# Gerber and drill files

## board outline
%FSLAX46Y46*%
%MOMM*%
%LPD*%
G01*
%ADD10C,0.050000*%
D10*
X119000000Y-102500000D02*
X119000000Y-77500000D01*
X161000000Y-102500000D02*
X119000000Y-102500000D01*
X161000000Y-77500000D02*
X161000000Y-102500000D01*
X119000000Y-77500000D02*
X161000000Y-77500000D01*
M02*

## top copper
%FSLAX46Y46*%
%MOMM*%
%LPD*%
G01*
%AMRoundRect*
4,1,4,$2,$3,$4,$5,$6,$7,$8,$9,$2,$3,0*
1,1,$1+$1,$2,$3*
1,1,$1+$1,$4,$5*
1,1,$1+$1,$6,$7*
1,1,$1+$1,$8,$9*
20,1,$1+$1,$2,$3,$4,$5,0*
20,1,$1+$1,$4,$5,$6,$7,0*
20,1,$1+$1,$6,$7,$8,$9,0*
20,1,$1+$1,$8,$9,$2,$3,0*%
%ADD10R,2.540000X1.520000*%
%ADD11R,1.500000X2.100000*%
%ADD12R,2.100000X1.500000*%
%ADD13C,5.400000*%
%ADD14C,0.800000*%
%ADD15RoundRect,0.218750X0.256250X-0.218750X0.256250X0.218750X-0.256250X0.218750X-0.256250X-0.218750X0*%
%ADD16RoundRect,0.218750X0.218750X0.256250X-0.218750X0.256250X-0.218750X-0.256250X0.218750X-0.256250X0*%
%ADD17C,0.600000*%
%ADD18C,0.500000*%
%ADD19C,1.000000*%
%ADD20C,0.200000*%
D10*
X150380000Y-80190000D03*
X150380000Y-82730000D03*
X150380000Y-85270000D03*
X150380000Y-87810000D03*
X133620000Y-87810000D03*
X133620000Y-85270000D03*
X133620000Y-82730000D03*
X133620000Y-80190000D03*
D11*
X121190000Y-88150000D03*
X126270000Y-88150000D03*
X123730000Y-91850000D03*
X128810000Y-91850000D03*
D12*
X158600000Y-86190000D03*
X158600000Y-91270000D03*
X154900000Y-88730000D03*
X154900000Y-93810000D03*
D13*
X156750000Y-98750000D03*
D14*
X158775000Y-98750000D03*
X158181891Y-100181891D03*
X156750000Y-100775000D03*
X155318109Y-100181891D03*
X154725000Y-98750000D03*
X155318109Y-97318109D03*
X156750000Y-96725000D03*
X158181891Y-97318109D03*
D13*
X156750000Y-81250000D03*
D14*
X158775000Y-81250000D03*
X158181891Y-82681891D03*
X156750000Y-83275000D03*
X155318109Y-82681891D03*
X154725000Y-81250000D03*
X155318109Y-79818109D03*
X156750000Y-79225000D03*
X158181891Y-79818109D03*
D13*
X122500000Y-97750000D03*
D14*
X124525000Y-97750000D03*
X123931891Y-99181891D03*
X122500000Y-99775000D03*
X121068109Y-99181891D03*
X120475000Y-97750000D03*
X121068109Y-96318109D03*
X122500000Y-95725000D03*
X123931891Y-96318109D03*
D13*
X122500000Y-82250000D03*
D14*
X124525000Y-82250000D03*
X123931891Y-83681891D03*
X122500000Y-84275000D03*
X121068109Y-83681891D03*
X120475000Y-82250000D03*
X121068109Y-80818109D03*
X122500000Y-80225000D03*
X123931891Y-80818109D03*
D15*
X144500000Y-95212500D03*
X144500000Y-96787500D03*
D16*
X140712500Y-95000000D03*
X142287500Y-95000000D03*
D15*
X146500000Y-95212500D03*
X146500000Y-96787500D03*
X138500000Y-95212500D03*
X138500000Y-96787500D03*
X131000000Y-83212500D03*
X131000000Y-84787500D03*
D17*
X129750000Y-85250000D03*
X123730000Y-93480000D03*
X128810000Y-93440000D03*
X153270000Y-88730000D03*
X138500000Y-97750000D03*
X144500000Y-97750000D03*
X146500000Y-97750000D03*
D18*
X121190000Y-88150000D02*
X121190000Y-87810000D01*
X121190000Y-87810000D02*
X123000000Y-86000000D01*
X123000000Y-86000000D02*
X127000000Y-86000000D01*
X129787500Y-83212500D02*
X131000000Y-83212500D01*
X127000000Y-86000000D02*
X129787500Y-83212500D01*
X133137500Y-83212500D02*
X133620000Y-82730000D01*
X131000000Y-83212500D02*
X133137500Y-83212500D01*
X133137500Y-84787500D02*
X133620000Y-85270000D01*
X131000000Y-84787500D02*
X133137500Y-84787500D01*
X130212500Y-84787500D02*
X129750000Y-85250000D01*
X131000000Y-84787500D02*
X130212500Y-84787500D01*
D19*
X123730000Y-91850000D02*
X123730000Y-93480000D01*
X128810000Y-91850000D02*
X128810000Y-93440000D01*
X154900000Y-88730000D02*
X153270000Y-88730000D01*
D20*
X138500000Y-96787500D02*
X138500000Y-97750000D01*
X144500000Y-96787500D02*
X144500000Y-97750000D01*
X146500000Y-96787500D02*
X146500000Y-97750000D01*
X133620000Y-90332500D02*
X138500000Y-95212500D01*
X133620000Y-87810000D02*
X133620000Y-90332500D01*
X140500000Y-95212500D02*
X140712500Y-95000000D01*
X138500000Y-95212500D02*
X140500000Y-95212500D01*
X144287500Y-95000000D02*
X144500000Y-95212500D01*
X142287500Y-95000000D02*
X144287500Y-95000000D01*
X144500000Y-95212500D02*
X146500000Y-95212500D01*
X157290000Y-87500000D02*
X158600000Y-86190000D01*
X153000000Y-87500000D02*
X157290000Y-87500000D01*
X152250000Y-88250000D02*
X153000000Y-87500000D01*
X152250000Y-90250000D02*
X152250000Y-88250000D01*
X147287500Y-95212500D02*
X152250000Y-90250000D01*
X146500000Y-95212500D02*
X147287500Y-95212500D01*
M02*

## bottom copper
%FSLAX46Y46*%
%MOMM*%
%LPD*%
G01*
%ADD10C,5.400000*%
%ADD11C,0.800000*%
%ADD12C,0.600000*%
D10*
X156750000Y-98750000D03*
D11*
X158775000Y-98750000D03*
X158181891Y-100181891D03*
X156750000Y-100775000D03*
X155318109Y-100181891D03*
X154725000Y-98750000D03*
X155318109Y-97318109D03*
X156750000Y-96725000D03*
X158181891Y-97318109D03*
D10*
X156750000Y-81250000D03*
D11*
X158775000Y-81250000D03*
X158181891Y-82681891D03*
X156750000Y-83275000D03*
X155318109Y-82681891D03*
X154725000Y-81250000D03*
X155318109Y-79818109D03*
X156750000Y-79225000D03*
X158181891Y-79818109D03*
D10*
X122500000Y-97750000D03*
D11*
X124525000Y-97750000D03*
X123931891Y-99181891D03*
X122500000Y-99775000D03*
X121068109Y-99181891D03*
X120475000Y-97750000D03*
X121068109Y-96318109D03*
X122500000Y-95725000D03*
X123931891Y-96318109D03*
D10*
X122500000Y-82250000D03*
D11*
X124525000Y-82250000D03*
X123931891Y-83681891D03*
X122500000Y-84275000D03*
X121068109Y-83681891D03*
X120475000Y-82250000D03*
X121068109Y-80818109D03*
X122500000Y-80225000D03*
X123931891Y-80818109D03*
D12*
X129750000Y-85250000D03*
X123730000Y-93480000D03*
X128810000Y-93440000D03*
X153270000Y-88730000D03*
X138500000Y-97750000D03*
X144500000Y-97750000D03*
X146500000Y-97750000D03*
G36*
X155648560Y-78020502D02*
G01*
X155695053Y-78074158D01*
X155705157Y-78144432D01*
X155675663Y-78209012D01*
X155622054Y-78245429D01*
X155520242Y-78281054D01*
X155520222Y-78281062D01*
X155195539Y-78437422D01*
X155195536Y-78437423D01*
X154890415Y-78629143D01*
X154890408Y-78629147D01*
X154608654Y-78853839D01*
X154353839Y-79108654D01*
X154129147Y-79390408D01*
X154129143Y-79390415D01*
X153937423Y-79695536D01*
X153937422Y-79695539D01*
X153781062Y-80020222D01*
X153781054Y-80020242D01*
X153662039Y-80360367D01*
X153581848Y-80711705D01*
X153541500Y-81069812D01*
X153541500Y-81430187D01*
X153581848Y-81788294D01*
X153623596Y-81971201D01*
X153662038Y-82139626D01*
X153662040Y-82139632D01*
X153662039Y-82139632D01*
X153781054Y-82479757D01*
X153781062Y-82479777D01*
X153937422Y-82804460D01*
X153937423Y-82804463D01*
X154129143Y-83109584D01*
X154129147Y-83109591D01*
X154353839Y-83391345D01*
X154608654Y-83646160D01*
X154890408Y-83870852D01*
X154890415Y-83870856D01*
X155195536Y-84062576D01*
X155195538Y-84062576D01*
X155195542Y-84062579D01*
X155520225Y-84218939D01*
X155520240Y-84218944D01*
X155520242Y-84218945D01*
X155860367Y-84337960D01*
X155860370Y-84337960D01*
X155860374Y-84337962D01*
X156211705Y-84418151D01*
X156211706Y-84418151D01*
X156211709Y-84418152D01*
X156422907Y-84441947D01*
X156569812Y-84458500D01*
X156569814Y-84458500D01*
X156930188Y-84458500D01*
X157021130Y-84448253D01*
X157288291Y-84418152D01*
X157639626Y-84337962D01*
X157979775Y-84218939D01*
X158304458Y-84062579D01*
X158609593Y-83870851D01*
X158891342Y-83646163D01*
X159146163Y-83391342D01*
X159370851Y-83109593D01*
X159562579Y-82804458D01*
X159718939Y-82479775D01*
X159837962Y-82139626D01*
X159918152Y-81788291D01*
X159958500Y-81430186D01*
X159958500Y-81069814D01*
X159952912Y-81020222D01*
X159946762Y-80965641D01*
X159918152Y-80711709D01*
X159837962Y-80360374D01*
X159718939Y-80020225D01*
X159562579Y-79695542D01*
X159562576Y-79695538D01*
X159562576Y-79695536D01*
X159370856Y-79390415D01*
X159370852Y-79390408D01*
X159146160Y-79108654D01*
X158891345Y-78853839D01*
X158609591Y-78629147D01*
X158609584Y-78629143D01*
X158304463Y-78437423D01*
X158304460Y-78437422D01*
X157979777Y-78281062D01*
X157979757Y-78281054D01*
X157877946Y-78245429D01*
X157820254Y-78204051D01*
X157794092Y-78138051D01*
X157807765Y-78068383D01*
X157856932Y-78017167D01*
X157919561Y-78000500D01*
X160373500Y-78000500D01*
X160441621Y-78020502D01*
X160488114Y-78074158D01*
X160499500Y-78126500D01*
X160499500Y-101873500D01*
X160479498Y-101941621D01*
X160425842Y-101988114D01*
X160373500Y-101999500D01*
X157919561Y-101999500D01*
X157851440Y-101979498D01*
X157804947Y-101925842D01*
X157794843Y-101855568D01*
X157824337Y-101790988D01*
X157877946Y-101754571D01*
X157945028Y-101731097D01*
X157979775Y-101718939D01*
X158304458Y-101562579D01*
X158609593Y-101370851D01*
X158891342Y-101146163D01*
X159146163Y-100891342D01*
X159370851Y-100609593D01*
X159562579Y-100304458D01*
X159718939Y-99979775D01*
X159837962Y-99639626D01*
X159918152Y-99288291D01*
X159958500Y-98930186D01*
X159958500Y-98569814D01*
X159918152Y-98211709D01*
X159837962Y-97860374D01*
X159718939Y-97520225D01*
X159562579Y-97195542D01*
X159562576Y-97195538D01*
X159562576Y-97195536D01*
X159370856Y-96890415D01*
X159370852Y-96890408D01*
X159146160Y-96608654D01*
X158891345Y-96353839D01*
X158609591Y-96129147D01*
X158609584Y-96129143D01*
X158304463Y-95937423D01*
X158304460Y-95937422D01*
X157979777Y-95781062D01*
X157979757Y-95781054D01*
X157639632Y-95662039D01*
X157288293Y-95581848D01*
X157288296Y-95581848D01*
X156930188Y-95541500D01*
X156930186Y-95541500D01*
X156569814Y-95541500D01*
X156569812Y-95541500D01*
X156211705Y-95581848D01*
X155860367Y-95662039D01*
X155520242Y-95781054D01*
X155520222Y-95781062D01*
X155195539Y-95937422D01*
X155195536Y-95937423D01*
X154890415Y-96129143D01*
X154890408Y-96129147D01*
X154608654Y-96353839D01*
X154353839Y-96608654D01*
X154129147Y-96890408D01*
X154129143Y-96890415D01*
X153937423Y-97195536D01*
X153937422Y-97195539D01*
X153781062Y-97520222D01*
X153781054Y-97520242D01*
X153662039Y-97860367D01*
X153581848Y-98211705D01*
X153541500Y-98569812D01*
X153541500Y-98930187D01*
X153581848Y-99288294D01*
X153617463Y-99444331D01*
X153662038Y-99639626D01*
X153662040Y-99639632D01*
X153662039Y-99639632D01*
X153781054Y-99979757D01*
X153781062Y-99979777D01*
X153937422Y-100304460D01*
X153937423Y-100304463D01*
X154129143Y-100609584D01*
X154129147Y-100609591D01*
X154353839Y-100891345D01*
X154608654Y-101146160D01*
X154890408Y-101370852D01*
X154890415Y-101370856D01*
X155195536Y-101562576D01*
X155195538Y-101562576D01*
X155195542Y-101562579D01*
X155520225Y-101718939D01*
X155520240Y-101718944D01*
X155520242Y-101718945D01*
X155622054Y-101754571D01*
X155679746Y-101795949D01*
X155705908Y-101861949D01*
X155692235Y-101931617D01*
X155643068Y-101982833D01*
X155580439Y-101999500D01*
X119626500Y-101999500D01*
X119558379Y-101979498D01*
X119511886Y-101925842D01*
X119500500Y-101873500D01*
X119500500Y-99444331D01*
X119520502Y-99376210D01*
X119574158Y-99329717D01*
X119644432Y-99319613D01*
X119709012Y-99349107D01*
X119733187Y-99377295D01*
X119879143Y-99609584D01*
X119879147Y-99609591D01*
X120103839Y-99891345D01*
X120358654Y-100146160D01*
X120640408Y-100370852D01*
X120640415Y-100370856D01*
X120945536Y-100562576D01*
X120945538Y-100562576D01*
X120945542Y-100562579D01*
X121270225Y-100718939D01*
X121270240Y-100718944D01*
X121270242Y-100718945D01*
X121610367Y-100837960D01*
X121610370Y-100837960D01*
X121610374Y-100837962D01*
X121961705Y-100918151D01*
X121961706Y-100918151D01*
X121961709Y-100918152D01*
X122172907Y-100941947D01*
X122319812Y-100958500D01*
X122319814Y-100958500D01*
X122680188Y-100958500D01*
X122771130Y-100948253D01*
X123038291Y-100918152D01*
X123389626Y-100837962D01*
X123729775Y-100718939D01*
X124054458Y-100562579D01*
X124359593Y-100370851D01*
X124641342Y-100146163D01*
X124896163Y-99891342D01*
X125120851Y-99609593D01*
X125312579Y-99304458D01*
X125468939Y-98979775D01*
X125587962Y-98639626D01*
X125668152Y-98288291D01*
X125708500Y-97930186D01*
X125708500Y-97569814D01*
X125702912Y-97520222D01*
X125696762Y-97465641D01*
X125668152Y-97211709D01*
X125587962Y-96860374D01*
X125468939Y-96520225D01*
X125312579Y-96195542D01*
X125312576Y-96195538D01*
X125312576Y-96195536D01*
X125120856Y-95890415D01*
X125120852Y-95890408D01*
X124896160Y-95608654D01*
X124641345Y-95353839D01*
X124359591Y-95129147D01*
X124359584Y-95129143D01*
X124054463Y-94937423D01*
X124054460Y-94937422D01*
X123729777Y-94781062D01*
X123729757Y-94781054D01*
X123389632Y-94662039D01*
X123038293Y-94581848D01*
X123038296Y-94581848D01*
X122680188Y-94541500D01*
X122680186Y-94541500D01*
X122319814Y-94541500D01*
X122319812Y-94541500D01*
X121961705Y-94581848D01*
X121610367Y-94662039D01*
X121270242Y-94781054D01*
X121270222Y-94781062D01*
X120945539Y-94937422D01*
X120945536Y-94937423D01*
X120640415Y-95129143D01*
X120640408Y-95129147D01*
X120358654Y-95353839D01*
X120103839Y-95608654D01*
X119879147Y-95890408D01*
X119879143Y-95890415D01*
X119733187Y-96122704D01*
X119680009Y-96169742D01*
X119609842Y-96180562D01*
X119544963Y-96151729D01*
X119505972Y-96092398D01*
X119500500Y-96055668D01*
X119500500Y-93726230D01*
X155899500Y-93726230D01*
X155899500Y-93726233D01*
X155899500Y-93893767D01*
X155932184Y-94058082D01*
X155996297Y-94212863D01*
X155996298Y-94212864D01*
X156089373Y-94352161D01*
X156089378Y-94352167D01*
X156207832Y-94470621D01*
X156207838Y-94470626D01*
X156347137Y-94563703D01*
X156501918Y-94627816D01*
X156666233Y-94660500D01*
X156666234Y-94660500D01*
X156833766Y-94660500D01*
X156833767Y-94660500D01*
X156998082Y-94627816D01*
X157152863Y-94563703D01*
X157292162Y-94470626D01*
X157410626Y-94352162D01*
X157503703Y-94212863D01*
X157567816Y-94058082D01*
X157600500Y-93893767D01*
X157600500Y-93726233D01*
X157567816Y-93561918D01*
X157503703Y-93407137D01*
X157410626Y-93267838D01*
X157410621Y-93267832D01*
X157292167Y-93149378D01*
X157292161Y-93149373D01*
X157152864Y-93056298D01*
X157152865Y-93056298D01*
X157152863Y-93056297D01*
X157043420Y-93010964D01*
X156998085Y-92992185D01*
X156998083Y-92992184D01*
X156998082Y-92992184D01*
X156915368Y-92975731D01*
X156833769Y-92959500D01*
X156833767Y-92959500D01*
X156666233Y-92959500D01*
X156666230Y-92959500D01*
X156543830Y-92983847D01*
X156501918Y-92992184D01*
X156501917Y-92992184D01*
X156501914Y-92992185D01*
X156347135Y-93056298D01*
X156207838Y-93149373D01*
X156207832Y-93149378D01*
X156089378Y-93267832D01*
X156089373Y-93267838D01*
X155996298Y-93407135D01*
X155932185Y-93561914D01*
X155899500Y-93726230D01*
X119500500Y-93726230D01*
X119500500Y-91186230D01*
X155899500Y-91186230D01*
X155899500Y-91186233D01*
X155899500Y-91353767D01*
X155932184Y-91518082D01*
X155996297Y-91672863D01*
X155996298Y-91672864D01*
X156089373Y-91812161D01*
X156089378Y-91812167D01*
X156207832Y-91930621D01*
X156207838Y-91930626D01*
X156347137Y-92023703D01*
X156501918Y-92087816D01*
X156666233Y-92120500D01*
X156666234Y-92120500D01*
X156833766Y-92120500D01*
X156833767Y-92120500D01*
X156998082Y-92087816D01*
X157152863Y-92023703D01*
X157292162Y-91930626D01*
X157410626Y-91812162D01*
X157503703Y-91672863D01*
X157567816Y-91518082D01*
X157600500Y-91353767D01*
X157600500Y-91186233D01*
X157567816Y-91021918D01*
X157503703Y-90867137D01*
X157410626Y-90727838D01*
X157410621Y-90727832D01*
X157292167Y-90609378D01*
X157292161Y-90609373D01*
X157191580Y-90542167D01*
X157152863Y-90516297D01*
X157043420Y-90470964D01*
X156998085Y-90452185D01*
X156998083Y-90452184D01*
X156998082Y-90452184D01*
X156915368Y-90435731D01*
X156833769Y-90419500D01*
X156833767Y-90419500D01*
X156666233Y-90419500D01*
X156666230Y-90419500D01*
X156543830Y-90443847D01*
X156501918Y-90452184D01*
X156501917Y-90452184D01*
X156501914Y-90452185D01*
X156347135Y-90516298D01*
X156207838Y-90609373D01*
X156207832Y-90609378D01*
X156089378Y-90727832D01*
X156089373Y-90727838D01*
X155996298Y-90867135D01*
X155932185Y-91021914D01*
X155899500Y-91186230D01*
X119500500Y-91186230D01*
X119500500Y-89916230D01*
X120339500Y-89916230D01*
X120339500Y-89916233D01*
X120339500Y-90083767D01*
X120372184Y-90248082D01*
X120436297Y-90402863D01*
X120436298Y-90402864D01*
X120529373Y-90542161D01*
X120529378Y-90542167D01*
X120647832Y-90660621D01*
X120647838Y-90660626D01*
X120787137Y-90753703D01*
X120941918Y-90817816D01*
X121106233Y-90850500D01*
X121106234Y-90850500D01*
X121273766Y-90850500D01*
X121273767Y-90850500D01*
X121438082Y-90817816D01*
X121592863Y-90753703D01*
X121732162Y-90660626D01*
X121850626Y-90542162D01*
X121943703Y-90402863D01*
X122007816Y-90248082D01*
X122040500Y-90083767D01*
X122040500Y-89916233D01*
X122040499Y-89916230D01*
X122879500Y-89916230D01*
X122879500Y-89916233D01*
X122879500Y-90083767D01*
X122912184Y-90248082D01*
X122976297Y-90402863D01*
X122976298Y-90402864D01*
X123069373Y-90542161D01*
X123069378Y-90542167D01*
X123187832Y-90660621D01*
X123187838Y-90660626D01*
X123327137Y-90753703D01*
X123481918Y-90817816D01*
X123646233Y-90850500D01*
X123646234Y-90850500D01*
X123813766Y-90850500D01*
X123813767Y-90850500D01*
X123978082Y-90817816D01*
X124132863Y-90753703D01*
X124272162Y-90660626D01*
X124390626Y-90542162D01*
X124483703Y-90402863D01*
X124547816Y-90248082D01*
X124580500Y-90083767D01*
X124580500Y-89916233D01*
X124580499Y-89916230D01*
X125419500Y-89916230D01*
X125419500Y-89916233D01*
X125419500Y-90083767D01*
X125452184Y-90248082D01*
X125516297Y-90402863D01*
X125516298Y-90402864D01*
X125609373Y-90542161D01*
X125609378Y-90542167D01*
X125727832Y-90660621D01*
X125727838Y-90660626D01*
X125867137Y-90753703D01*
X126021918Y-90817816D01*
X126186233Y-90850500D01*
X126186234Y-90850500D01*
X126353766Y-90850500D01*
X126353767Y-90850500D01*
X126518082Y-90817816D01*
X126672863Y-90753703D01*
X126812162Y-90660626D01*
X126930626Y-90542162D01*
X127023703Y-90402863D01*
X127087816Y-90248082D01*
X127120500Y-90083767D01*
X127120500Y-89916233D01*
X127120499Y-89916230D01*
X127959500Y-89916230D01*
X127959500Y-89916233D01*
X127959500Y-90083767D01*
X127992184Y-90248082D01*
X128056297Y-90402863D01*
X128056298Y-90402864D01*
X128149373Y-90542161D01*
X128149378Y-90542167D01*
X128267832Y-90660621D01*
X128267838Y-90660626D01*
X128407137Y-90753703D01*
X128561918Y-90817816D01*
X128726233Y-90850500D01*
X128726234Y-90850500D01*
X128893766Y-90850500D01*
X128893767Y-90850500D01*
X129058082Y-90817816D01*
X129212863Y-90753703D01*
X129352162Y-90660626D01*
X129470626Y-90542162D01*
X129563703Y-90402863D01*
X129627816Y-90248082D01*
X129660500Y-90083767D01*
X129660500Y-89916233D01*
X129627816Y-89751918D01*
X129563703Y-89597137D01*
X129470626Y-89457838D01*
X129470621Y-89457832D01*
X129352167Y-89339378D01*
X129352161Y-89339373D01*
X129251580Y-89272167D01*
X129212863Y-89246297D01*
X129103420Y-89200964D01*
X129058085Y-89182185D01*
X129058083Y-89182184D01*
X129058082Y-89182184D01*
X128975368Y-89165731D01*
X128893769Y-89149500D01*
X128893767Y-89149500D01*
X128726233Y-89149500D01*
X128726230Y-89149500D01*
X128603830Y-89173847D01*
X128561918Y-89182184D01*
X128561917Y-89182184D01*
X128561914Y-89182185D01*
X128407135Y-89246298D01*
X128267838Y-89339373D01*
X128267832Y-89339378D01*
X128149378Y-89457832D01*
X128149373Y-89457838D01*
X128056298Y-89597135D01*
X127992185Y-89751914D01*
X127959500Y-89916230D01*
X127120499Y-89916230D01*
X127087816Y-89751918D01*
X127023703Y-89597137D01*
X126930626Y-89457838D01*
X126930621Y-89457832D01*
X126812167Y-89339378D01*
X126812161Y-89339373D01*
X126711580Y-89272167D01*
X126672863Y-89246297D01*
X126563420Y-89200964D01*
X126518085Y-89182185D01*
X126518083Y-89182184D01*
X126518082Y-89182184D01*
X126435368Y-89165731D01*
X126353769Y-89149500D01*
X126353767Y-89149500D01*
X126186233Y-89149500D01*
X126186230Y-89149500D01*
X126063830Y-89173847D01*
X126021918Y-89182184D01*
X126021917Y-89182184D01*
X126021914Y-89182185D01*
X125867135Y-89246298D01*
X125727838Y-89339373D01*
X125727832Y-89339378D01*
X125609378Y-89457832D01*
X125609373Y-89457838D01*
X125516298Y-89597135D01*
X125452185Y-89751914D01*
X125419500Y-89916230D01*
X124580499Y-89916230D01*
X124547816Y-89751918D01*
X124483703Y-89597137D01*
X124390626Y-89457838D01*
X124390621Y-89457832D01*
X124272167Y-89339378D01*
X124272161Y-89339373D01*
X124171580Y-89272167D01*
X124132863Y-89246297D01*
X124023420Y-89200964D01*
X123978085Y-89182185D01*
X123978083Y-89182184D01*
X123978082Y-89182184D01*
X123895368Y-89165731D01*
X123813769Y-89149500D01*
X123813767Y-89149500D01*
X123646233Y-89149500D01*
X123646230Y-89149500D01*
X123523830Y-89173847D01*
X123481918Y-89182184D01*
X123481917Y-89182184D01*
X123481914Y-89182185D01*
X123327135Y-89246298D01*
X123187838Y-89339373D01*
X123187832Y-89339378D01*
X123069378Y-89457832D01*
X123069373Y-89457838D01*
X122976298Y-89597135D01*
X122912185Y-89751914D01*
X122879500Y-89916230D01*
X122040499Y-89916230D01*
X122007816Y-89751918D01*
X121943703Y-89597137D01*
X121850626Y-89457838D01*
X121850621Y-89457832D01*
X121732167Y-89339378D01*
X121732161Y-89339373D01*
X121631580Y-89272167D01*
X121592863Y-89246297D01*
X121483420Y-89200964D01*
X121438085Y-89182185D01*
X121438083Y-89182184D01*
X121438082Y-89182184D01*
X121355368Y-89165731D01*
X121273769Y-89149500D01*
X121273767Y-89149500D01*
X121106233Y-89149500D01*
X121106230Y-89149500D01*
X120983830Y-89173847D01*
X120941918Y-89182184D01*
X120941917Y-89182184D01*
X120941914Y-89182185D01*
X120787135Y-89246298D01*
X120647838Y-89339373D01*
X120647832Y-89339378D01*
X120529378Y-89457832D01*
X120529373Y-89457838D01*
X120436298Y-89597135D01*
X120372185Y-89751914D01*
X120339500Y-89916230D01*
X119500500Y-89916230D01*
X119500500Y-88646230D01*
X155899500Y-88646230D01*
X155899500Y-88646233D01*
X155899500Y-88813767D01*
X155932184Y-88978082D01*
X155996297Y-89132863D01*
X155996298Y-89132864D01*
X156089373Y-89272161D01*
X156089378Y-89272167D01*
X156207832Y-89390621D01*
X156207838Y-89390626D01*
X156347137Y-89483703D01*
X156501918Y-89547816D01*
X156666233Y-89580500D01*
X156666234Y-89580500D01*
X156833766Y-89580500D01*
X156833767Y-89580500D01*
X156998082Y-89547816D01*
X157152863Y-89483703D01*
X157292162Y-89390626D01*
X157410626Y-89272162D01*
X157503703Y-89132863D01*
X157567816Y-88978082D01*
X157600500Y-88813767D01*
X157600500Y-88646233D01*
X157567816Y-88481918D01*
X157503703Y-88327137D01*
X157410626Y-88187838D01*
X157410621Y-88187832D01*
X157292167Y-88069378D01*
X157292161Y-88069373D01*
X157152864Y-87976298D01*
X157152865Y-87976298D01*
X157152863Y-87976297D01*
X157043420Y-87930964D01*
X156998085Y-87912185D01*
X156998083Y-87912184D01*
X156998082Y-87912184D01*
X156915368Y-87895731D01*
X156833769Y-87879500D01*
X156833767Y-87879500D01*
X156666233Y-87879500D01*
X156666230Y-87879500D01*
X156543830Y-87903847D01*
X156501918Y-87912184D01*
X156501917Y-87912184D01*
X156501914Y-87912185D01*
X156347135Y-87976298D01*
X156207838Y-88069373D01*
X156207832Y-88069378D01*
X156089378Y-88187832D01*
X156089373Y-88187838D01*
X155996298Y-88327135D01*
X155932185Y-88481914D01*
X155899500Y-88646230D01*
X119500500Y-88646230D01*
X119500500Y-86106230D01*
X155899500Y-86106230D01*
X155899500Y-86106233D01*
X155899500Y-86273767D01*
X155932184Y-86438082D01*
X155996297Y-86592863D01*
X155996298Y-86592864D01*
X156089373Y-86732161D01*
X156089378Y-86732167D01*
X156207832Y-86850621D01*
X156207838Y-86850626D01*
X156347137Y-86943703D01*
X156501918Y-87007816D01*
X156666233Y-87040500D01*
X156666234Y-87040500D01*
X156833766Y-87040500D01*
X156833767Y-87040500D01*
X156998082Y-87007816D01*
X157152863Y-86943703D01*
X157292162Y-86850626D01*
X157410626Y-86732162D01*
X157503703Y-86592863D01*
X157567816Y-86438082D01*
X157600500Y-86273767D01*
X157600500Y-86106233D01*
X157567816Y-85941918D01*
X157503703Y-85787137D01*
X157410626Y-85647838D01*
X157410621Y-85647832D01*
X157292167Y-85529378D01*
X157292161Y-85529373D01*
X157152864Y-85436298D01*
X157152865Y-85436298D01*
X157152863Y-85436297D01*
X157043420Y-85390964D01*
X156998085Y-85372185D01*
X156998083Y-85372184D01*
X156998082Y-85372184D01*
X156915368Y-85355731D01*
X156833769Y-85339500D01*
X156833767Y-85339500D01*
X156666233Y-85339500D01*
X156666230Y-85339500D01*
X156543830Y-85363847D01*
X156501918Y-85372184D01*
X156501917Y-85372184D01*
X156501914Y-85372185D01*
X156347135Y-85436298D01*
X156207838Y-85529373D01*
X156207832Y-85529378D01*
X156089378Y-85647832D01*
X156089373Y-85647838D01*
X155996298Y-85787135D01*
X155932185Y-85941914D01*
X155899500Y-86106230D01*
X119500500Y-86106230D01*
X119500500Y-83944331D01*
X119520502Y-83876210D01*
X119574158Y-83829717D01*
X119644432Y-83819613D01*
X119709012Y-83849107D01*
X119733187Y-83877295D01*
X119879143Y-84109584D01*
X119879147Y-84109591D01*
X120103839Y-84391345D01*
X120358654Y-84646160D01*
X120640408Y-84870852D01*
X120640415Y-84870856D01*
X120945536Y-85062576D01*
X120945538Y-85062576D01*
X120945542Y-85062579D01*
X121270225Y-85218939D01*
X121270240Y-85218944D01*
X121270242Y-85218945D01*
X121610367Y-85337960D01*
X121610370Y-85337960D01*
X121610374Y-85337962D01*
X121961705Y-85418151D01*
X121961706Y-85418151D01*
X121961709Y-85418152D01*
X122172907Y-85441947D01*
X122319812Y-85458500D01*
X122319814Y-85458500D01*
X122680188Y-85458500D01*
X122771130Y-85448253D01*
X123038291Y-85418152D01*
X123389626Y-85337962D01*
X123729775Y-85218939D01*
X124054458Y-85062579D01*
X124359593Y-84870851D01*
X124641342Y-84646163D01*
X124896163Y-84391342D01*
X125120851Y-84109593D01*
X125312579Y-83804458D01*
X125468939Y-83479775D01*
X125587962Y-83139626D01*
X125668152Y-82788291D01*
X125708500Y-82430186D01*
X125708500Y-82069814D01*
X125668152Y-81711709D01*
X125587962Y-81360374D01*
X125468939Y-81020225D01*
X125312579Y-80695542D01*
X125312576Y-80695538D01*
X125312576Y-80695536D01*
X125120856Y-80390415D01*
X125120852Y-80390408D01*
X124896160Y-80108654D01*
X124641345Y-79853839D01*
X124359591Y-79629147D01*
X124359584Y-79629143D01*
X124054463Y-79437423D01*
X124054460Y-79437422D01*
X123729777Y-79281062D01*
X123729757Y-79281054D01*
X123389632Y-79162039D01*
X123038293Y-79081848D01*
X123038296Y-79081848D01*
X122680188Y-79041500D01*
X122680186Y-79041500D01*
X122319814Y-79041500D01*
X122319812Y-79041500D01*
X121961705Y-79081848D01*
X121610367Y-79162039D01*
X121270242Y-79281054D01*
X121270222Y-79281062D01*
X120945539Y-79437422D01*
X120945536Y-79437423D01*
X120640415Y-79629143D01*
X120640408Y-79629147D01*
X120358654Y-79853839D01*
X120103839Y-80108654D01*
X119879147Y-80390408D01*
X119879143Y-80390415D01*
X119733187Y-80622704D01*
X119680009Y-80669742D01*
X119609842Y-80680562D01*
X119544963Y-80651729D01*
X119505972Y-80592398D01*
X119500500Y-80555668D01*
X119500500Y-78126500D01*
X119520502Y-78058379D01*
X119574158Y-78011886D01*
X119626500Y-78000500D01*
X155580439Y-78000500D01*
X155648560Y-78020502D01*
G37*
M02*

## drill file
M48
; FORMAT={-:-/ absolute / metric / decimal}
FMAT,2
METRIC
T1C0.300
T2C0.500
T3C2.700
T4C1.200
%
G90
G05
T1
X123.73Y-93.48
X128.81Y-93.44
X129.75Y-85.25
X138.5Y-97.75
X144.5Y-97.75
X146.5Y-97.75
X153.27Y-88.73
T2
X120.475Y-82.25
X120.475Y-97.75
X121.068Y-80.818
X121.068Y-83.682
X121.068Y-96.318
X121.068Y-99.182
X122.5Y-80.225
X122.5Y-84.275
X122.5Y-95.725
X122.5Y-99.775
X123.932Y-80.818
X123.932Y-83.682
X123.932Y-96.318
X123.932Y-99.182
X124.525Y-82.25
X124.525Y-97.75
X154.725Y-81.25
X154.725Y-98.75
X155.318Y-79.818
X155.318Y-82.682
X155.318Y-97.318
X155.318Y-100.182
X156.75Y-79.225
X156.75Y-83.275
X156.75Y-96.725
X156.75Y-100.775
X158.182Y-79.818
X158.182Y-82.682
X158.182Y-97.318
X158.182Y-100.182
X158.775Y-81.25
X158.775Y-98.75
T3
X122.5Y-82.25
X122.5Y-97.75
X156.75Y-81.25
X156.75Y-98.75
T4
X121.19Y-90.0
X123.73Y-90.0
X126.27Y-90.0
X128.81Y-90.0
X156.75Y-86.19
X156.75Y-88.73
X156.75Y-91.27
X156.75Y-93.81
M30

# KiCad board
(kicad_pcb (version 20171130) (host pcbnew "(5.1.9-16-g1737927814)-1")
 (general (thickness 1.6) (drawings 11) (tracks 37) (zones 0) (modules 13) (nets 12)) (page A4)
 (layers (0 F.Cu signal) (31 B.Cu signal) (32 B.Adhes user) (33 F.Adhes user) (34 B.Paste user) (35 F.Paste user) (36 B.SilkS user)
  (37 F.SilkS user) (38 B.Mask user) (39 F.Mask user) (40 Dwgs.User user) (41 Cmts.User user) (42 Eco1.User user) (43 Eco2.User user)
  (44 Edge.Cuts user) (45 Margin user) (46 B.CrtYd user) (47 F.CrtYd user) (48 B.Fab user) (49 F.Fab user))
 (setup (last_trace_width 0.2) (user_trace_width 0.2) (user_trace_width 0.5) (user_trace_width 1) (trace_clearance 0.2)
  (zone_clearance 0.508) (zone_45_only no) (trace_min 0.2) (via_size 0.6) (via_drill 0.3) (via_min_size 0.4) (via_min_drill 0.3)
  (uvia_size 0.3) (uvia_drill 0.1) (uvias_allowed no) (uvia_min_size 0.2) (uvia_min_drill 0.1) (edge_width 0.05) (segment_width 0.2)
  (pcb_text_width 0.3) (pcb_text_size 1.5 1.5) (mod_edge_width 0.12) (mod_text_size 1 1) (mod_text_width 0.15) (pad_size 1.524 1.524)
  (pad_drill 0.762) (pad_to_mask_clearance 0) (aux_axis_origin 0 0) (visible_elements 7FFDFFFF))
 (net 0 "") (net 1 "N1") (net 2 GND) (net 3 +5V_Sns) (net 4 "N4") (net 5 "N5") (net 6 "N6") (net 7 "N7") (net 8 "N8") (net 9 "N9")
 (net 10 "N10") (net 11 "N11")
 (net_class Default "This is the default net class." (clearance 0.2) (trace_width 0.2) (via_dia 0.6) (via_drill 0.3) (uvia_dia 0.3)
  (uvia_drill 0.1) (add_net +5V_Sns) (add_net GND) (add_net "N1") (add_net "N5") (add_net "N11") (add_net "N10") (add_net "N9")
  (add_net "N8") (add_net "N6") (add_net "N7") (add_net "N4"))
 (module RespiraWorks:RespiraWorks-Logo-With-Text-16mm (layer B.Cu) (at 139.5 89.75 180)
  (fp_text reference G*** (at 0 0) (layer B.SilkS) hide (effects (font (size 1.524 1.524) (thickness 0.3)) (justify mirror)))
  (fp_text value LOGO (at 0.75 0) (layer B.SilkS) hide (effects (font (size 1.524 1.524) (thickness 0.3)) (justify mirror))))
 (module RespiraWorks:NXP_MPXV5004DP (layer F.Cu) (at 142 84)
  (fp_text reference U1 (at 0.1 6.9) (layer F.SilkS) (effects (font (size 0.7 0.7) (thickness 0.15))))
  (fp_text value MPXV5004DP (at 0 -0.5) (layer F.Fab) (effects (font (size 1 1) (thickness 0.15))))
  (pad 8 smd rect (at 8.38 -3.81) (size 2.54 1.52) (layers F.Cu F.Paste F.Mask))
  (pad 7 smd rect (at 8.38 -1.27) (size 2.54 1.52) (layers F.Cu F.Paste F.Mask))
  (pad 6 smd rect (at 8.38 1.27) (size 2.54 1.52) (layers F.Cu F.Paste F.Mask))
  (pad 5 smd rect (at 8.38 3.81) (size 2.54 1.52) (layers F.Cu F.Paste F.Mask))
  (pad 4 smd rect (at -8.38 3.81) (size 2.54 1.52) (layers F.Cu F.Paste F.Mask) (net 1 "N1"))
  (pad 3 smd rect (at -8.38 1.27) (size 2.54 1.52) (layers F.Cu F.Paste F.Mask) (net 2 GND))
  (pad 2 smd rect (at -8.38 -1.27) (size 2.54 1.52) (layers F.Cu F.Paste F.Mask) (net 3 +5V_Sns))
  (pad 1 smd rect (at -8.38 -3.81) (size 2.54 1.52) (layers F.Cu F.Paste F.Mask)))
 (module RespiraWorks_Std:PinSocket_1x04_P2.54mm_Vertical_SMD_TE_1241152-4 (layer F.Cu) (at 125 90 90)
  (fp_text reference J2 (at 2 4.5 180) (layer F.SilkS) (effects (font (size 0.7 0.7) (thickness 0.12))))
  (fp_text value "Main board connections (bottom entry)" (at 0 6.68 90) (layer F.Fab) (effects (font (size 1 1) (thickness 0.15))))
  (pad "" np_thru_hole circle (at 0 1.27 90) (size 1.2 1.2) (drill 1.2) (layers *.Cu *.Mask))
  (pad "" np_thru_hole circle (at 0 -1.27 90) (size 1.2 1.2) (drill 1.2) (layers *.Cu *.Mask))
  (pad "" np_thru_hole circle (at 0 -3.81 90) (size 1.2 1.2) (drill 1.2) (layers *.Cu *.Mask))
  (pad 1 smd rect (at 1.85 -3.81 90) (size 2.1 1.5) (layers F.Cu F.Paste F.Mask) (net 3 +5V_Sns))
  (pad 3 smd rect (at 1.85 1.27 90) (size 2.1 1.5) (layers F.Cu F.Paste F.Mask) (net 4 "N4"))
  (pad 2 smd rect (at -1.85 -1.27 90) (size 2.1 1.5) (layers F.Cu F.Paste F.Mask) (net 2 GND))
  (pad 4 smd rect (at -1.85 3.81 90) (size 2.1 1.5) (layers F.Cu F.Paste F.Mask) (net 2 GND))
  (pad "" np_thru_hole circle (at 0 3.81 90) (size 1.2 1.2) (drill 1.2) (layers *.Cu *.Mask)))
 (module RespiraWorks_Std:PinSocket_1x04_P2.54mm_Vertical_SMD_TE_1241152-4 (layer F.Cu) (at 156.75 90)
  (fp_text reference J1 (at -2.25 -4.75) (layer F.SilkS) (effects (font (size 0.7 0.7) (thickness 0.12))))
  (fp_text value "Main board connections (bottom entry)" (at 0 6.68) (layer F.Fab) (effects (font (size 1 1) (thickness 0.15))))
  (pad "" np_thru_hole circle (at 0 1.27) (size 1.2 1.2) (drill 1.2) (layers *.Cu *.Mask))
  (pad "" np_thru_hole circle (at 0 -1.27) (size 1.2 1.2) (drill 1.2) (layers *.Cu *.Mask))
  (pad "" np_thru_hole circle (at 0 -3.81) (size 1.2 1.2) (drill 1.2) (layers *.Cu *.Mask))
  (pad 1 smd rect (at 1.85 -3.81) (size 2.1 1.5) (layers F.Cu F.Paste F.Mask) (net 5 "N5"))
  (pad 3 smd rect (at 1.85 1.27) (size 2.1 1.5) (layers F.Cu F.Paste F.Mask) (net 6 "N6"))
  (pad 2 smd rect (at -1.85 -1.27) (size 2.1 1.5) (layers F.Cu F.Paste F.Mask) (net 2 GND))
  (pad 4 smd rect (at -1.85 3.81) (size 2.1 1.5) (layers F.Cu F.Paste F.Mask) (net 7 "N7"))
  (pad "" np_thru_hole circle (at 0 3.81) (size 1.2 1.2) (drill 1.2) (layers *.Cu *.Mask)))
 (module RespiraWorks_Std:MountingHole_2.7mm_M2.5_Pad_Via (layer F.Cu) (at 156.75 98.75)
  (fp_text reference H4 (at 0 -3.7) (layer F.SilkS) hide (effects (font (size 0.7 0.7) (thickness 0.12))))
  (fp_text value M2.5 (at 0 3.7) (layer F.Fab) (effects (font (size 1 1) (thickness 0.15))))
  (pad 1 thru_hole circle (at 0 0) (size 5.4 5.4) (drill 2.7) (layers *.Cu *.Mask) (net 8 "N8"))
  (pad 1 thru_hole circle (at 2.025 0) (size 0.8 0.8) (drill 0.5) (layers *.Cu *.Mask) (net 8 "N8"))
  (pad 1 thru_hole circle (at 1.431891 1.431891) (size 0.8 0.8) (drill 0.5) (layers *.Cu *.Mask) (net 8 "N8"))
  (pad 1 thru_hole circle (at 0 2.025) (size 0.8 0.8) (drill 0.5) (layers *.Cu *.Mask) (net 8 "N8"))
  (pad 1 thru_hole circle (at -1.431891 1.431891) (size 0.8 0.8) (drill 0.5) (layers *.Cu *.Mask) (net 8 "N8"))
  (pad 1 thru_hole circle (at -2.025 0) (size 0.8 0.8) (drill 0.5) (layers *.Cu *.Mask) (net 8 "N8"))
  (pad 1 thru_hole circle (at -1.431891 -1.431891) (size 0.8 0.8) (drill 0.5) (layers *.Cu *.Mask) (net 8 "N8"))
  (pad 1 thru_hole circle (at 0 -2.025) (size 0.8 0.8) (drill 0.5) (layers *.Cu *.Mask) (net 8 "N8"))
  (pad 1 thru_hole circle (at 1.431891 -1.431891) (size 0.8 0.8) (drill 0.5) (layers *.Cu *.Mask) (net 8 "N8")))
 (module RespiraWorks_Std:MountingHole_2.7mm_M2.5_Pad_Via (layer F.Cu) (at 156.75 81.25)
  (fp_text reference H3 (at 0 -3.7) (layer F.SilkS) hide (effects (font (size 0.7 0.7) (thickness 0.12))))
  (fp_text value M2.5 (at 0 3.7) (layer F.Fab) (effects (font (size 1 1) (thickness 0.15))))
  (pad 1 thru_hole circle (at 0 0) (size 5.4 5.4) (drill 2.7) (layers *.Cu *.Mask) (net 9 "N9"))
  (pad 1 thru_hole circle (at 2.025 0) (size 0.8 0.8) (drill 0.5) (layers *.Cu *.Mask) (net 9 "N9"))
  (pad 1 thru_hole circle (at 1.431891 1.431891) (size 0.8 0.8) (drill 0.5) (layers *.Cu *.Mask) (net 9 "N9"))
  (pad 1 thru_hole circle (at 0 2.025) (size 0.8 0.8) (drill 0.5) (layers *.Cu *.Mask) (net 9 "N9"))
  (pad 1 thru_hole circle (at -1.431891 1.431891) (size 0.8 0.8) (drill 0.5) (layers *.Cu *.Mask) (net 9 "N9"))
  (pad 1 thru_hole circle (at -2.025 0) (size 0.8 0.8) (drill 0.5) (layers *.Cu *.Mask) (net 9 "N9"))
  (pad 1 thru_hole circle (at -1.431891 -1.431891) (size 0.8 0.8) (drill 0.5) (layers *.Cu *.Mask) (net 9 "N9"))
  (pad 1 thru_hole circle (at 0 -2.025) (size 0.8 0.8) (drill 0.5) (layers *.Cu *.Mask) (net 9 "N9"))
  (pad 1 thru_hole circle (at 1.431891 -1.431891) (size 0.8 0.8) (drill 0.5) (layers *.Cu *.Mask) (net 9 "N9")))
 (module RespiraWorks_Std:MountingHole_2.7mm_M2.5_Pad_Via (layer F.Cu) (at 122.5 97.75)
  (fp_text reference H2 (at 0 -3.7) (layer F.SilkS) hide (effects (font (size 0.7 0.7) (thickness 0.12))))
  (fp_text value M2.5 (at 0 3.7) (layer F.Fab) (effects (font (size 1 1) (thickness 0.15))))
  (pad 1 thru_hole circle (at 0 0) (size 5.4 5.4) (drill 2.7) (layers *.Cu *.Mask) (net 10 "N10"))
  (pad 1 thru_hole circle (at 2.025 0) (size 0.8 0.8) (drill 0.5) (layers *.Cu *.Mask) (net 10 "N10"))
  (pad 1 thru_hole circle (at 1.431891 1.431891) (size 0.8 0.8) (drill 0.5) (layers *.Cu *.Mask) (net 10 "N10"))
  (pad 1 thru_hole circle (at 0 2.025) (size 0.8 0.8) (drill 0.5) (layers *.Cu *.Mask) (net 10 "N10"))
  (pad 1 thru_hole circle (at -1.431891 1.431891) (size 0.8 0.8) (drill 0.5) (layers *.Cu *.Mask) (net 10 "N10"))
  (pad 1 thru_hole circle (at -2.025 0) (size 0.8 0.8) (drill 0.5) (layers *.Cu *.Mask) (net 10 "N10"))
  (pad 1 thru_hole circle (at -1.431891 -1.431891) (size 0.8 0.8) (drill 0.5) (layers *.Cu *.Mask) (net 10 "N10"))
  (pad 1 thru_hole circle (at 0 -2.025) (size 0.8 0.8) (drill 0.5) (layers *.Cu *.Mask) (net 10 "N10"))
  (pad 1 thru_hole circle (at 1.431891 -1.431891) (size 0.8 0.8) (drill 0.5) (layers *.Cu *.Mask) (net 10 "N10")))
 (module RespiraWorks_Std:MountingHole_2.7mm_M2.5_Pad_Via (layer F.Cu) (at 122.5 82.25)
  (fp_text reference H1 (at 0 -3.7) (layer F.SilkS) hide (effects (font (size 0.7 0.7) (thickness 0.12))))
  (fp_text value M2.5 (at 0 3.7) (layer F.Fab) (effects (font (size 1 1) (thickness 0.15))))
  (pad 1 thru_hole circle (at 0 0) (size 5.4 5.4) (drill 2.7) (layers *.Cu *.Mask) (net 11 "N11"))
  (pad 1 thru_hole circle (at 2.025 0) (size 0.8 0.8) (drill 0.5) (layers *.Cu *.Mask) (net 11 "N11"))
  (pad 1 thru_hole circle (at 1.431891 1.431891) (size 0.8 0.8) (drill 0.5) (layers *.Cu *.Mask) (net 11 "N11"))
  (pad 1 thru_hole circle (at 0 2.025) (size 0.8 0.8) (drill 0.5) (layers *.Cu *.Mask) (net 11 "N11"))
  (pad 1 thru_hole circle (at -1.431891 1.431891) (size 0.8 0.8) (drill 0.5) (layers *.Cu *.Mask) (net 11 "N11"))
  (pad 1 thru_hole circle (at -2.025 0) (size 0.8 0.8) (drill 0.5) (layers *.Cu *.Mask) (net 11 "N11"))
  (pad 1 thru_hole circle (at -1.431891 -1.431891) (size 0.8 0.8) (drill 0.5) (layers *.Cu *.Mask) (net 11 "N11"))
  (pad 1 thru_hole circle (at 0 -2.025) (size 0.8 0.8) (drill 0.5) (layers *.Cu *.Mask) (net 11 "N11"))
  (pad 1 thru_hole circle (at 1.431891 -1.431891) (size 0.8 0.8) (drill 0.5) (layers *.Cu *.Mask) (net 11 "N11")))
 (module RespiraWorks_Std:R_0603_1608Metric (layer F.Cu) (at 144.5 96 90)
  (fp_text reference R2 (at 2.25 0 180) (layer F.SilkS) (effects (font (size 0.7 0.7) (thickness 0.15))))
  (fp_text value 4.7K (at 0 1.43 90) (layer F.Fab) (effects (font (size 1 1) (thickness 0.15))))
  (pad 2 smd roundrect (at 0.7875 0 90) (size 0.875 0.95) (layers F.Cu F.Paste F.Mask) (roundrect_rratio 0.25) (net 5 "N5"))
  (pad 1 smd roundrect (at -0.7875 0 90) (size 0.875 0.95) (layers F.Cu F.Paste F.Mask) (roundrect_rratio 0.25) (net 2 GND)))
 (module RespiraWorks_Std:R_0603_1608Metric (layer F.Cu) (at 141.5 95 180)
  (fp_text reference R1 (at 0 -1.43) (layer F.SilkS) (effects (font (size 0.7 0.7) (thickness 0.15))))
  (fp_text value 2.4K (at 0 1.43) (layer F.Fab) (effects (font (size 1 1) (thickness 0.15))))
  (pad 2 smd roundrect (at 0.7875 0 180) (size 0.875 0.95) (layers F.Cu F.Paste F.Mask) (roundrect_rratio 0.25) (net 1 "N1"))
  (pad 1 smd roundrect (at -0.7875 0 180) (size 0.875 0.95) (layers F.Cu F.Paste F.Mask) (roundrect_rratio 0.25) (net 5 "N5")))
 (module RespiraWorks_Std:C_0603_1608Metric (layer F.Cu) (at 146.5 96 90)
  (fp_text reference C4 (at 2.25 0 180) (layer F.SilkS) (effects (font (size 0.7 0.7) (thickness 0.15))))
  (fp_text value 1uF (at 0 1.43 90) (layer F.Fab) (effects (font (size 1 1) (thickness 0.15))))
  (pad 2 smd roundrect (at 0.7875 0 90) (size 0.875 0.95) (layers F.Cu F.Paste F.Mask) (roundrect_rratio 0.25) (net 5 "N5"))
  (pad 1 smd roundrect (at -0.7875 0 90) (size 0.875 0.95) (layers F.Cu F.Paste F.Mask) (roundrect_rratio 0.25) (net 2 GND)))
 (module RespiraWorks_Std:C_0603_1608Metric (layer F.Cu) (at 138.5 96 90)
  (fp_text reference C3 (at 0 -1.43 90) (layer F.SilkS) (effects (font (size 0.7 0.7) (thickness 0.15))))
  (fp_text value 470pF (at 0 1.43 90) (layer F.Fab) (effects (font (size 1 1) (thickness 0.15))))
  (pad 2 smd roundrect (at 0.7875 0 90) (size 0.875 0.95) (layers F.Cu F.Paste F.Mask) (roundrect_rratio 0.25) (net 1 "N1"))
  (pad 1 smd roundrect (at -0.7875 0 90) (size 0.875 0.95) (layers F.Cu F.Paste F.Mask) (roundrect_rratio 0.25) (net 2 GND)))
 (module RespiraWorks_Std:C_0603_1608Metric (layer F.Cu) (at 131 84 90)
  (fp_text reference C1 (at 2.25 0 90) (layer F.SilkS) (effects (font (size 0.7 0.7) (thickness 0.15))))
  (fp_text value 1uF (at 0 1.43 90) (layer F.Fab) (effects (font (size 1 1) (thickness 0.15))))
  (pad 2 smd roundrect (at 0.7875 0 90) (size 0.875 0.95) (layers F.Cu F.Paste F.Mask) (roundrect_rratio 0.25) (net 3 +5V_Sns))
  (pad 1 smd roundrect (at -0.7875 0 90) (size 0.875 0.95) (layers F.Cu F.Paste F.Mask) (roundrect_rratio 0.25) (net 2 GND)))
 (gr_line (start 119 102.5) (end 119 77.5) (layer Edge.Cuts) (width 0.05))
 (gr_line (start 161 102.5) (end 119 102.5) (layer Edge.Cuts) (width 0.05))
 (gr_line (start 161 77.5) (end 161 102.5) (layer Edge.Cuts) (width 0.05))
 (gr_line (start 119 77.5) (end 161 77.5) (layer Edge.Cuts) (width 0.05))
 (segment (start 121.19 88.15) (end 121.19 87.81) (width 0.5) (layer F.Cu) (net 3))
 (segment (start 121.19 87.81) (end 123 86) (width 0.5) (layer F.Cu) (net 3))
 (segment (start 123 86) (end 127 86) (width 0.5) (layer F.Cu) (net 3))
 (segment (start 129.7875 83.2125) (end 131 83.2125) (width 0.5) (layer F.Cu) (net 3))
 (segment (start 127 86) (end 129.7875 83.2125) (width 0.5) (layer F.Cu) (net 3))
 (segment (start 133.1375 83.2125) (end 133.62 82.73) (width 0.5) (layer F.Cu) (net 3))
 (segment (start 131 83.2125) (end 133.1375 83.2125) (width 0.5) (layer F.Cu) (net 3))
 (segment (start 133.1375 84.7875) (end 133.62 85.27) (width 0.5) (layer F.Cu) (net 2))
 (segment (start 131 84.7875) (end 133.1375 84.7875) (width 0.5) (layer F.Cu) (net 2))
 (via (at 129.75 85.25) (size 0.6) (drill 0.3) (layers F.Cu B.Cu) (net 2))
 (segment (start 130.2125 84.7875) (end 129.75 85.25) (width 0.5) (layer F.Cu) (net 2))
 (segment (start 131 84.7875) (end 130.2125 84.7875) (width 0.5) (layer F.Cu) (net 2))
 (segment (start 123.73 91.85) (end 123.73 93.48) (width 1) (layer F.Cu) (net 2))
 (via (at 123.73 93.48) (size 0.6) (drill 0.3) (layers F.Cu B.Cu) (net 2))
 (segment (start 128.81 91.85) (end 128.81 93.44) (width 1) (layer F.Cu) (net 2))
 (via (at 128.81 93.44) (size 0.6) (drill 0.3) (layers F.Cu B.Cu) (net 2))
 (segment (start 154.9 88.73) (end 153.27 88.73) (width 1) (layer F.Cu) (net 2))
 (via (at 153.27 88.73) (size 0.6) (drill 0.3) (layers F.Cu B.Cu) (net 2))
 (segment (start 138.5 96.7875) (end 138.5 97.75) (width 0.2) (layer F.Cu) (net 2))
 (via (at 138.5 97.75) (size 0.6) (drill 0.3) (layers F.Cu B.Cu) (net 2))
 (segment (start 144.5 96.7875) (end 144.5 97.75) (width 0.2) (layer F.Cu) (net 2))
 (via (at 144.5 97.75) (size 0.6) (drill 0.3) (layers F.Cu B.Cu) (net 2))
 (segment (start 146.5 96.7875) (end 146.5 97.75) (width 0.2) (layer F.Cu) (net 2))
 (via (at 146.5 97.75) (size 0.6) (drill 0.3) (layers F.Cu B.Cu) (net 2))
 (segment (start 133.62 90.3325) (end 138.5 95.2125) (width 0.2) (layer F.Cu) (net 1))
 (segment (start 133.62 87.81) (end 133.62 90.3325) (width 0.2) (layer F.Cu) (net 1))
 (segment (start 140.5 95.2125) (end 140.7125 95) (width 0.2) (layer F.Cu) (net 1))
 (segment (start 138.5 95.2125) (end 140.5 95.2125) (width 0.2) (layer F.Cu) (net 1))
 (segment (start 144.2875 95) (end 144.5 95.2125) (width 0.2) (layer F.Cu) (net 5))
 (segment (start 142.2875 95) (end 144.2875 95) (width 0.2) (layer F.Cu) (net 5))
 (segment (start 144.5 95.2125) (end 146.5 95.2125) (width 0.2) (layer F.Cu) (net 5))
 (segment (start 157.29 87.5) (end 158.6 86.19) (width 0.2) (layer F.Cu) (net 5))
 (segment (start 153 87.5) (end 157.29 87.5) (width 0.2) (layer F.Cu) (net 5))
 (segment (start 152.25 88.25) (end 153 87.5) (width 0.2) (layer F.Cu) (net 5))
 (segment (start 152.25 90.25) (end 152.25 88.25) (width 0.2) (layer F.Cu) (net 5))
 (segment (start 147.2875 95.2125) (end 152.25 90.25) (width 0.2) (layer F.Cu) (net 5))
 (segment (start 146.5 95.2125) (end 147.2875 95.2125) (width 0.2) (layer F.Cu) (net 5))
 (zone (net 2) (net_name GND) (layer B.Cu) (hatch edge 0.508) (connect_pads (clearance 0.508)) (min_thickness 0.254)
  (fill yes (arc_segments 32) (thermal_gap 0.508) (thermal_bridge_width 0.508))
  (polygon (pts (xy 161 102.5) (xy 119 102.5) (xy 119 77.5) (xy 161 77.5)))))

